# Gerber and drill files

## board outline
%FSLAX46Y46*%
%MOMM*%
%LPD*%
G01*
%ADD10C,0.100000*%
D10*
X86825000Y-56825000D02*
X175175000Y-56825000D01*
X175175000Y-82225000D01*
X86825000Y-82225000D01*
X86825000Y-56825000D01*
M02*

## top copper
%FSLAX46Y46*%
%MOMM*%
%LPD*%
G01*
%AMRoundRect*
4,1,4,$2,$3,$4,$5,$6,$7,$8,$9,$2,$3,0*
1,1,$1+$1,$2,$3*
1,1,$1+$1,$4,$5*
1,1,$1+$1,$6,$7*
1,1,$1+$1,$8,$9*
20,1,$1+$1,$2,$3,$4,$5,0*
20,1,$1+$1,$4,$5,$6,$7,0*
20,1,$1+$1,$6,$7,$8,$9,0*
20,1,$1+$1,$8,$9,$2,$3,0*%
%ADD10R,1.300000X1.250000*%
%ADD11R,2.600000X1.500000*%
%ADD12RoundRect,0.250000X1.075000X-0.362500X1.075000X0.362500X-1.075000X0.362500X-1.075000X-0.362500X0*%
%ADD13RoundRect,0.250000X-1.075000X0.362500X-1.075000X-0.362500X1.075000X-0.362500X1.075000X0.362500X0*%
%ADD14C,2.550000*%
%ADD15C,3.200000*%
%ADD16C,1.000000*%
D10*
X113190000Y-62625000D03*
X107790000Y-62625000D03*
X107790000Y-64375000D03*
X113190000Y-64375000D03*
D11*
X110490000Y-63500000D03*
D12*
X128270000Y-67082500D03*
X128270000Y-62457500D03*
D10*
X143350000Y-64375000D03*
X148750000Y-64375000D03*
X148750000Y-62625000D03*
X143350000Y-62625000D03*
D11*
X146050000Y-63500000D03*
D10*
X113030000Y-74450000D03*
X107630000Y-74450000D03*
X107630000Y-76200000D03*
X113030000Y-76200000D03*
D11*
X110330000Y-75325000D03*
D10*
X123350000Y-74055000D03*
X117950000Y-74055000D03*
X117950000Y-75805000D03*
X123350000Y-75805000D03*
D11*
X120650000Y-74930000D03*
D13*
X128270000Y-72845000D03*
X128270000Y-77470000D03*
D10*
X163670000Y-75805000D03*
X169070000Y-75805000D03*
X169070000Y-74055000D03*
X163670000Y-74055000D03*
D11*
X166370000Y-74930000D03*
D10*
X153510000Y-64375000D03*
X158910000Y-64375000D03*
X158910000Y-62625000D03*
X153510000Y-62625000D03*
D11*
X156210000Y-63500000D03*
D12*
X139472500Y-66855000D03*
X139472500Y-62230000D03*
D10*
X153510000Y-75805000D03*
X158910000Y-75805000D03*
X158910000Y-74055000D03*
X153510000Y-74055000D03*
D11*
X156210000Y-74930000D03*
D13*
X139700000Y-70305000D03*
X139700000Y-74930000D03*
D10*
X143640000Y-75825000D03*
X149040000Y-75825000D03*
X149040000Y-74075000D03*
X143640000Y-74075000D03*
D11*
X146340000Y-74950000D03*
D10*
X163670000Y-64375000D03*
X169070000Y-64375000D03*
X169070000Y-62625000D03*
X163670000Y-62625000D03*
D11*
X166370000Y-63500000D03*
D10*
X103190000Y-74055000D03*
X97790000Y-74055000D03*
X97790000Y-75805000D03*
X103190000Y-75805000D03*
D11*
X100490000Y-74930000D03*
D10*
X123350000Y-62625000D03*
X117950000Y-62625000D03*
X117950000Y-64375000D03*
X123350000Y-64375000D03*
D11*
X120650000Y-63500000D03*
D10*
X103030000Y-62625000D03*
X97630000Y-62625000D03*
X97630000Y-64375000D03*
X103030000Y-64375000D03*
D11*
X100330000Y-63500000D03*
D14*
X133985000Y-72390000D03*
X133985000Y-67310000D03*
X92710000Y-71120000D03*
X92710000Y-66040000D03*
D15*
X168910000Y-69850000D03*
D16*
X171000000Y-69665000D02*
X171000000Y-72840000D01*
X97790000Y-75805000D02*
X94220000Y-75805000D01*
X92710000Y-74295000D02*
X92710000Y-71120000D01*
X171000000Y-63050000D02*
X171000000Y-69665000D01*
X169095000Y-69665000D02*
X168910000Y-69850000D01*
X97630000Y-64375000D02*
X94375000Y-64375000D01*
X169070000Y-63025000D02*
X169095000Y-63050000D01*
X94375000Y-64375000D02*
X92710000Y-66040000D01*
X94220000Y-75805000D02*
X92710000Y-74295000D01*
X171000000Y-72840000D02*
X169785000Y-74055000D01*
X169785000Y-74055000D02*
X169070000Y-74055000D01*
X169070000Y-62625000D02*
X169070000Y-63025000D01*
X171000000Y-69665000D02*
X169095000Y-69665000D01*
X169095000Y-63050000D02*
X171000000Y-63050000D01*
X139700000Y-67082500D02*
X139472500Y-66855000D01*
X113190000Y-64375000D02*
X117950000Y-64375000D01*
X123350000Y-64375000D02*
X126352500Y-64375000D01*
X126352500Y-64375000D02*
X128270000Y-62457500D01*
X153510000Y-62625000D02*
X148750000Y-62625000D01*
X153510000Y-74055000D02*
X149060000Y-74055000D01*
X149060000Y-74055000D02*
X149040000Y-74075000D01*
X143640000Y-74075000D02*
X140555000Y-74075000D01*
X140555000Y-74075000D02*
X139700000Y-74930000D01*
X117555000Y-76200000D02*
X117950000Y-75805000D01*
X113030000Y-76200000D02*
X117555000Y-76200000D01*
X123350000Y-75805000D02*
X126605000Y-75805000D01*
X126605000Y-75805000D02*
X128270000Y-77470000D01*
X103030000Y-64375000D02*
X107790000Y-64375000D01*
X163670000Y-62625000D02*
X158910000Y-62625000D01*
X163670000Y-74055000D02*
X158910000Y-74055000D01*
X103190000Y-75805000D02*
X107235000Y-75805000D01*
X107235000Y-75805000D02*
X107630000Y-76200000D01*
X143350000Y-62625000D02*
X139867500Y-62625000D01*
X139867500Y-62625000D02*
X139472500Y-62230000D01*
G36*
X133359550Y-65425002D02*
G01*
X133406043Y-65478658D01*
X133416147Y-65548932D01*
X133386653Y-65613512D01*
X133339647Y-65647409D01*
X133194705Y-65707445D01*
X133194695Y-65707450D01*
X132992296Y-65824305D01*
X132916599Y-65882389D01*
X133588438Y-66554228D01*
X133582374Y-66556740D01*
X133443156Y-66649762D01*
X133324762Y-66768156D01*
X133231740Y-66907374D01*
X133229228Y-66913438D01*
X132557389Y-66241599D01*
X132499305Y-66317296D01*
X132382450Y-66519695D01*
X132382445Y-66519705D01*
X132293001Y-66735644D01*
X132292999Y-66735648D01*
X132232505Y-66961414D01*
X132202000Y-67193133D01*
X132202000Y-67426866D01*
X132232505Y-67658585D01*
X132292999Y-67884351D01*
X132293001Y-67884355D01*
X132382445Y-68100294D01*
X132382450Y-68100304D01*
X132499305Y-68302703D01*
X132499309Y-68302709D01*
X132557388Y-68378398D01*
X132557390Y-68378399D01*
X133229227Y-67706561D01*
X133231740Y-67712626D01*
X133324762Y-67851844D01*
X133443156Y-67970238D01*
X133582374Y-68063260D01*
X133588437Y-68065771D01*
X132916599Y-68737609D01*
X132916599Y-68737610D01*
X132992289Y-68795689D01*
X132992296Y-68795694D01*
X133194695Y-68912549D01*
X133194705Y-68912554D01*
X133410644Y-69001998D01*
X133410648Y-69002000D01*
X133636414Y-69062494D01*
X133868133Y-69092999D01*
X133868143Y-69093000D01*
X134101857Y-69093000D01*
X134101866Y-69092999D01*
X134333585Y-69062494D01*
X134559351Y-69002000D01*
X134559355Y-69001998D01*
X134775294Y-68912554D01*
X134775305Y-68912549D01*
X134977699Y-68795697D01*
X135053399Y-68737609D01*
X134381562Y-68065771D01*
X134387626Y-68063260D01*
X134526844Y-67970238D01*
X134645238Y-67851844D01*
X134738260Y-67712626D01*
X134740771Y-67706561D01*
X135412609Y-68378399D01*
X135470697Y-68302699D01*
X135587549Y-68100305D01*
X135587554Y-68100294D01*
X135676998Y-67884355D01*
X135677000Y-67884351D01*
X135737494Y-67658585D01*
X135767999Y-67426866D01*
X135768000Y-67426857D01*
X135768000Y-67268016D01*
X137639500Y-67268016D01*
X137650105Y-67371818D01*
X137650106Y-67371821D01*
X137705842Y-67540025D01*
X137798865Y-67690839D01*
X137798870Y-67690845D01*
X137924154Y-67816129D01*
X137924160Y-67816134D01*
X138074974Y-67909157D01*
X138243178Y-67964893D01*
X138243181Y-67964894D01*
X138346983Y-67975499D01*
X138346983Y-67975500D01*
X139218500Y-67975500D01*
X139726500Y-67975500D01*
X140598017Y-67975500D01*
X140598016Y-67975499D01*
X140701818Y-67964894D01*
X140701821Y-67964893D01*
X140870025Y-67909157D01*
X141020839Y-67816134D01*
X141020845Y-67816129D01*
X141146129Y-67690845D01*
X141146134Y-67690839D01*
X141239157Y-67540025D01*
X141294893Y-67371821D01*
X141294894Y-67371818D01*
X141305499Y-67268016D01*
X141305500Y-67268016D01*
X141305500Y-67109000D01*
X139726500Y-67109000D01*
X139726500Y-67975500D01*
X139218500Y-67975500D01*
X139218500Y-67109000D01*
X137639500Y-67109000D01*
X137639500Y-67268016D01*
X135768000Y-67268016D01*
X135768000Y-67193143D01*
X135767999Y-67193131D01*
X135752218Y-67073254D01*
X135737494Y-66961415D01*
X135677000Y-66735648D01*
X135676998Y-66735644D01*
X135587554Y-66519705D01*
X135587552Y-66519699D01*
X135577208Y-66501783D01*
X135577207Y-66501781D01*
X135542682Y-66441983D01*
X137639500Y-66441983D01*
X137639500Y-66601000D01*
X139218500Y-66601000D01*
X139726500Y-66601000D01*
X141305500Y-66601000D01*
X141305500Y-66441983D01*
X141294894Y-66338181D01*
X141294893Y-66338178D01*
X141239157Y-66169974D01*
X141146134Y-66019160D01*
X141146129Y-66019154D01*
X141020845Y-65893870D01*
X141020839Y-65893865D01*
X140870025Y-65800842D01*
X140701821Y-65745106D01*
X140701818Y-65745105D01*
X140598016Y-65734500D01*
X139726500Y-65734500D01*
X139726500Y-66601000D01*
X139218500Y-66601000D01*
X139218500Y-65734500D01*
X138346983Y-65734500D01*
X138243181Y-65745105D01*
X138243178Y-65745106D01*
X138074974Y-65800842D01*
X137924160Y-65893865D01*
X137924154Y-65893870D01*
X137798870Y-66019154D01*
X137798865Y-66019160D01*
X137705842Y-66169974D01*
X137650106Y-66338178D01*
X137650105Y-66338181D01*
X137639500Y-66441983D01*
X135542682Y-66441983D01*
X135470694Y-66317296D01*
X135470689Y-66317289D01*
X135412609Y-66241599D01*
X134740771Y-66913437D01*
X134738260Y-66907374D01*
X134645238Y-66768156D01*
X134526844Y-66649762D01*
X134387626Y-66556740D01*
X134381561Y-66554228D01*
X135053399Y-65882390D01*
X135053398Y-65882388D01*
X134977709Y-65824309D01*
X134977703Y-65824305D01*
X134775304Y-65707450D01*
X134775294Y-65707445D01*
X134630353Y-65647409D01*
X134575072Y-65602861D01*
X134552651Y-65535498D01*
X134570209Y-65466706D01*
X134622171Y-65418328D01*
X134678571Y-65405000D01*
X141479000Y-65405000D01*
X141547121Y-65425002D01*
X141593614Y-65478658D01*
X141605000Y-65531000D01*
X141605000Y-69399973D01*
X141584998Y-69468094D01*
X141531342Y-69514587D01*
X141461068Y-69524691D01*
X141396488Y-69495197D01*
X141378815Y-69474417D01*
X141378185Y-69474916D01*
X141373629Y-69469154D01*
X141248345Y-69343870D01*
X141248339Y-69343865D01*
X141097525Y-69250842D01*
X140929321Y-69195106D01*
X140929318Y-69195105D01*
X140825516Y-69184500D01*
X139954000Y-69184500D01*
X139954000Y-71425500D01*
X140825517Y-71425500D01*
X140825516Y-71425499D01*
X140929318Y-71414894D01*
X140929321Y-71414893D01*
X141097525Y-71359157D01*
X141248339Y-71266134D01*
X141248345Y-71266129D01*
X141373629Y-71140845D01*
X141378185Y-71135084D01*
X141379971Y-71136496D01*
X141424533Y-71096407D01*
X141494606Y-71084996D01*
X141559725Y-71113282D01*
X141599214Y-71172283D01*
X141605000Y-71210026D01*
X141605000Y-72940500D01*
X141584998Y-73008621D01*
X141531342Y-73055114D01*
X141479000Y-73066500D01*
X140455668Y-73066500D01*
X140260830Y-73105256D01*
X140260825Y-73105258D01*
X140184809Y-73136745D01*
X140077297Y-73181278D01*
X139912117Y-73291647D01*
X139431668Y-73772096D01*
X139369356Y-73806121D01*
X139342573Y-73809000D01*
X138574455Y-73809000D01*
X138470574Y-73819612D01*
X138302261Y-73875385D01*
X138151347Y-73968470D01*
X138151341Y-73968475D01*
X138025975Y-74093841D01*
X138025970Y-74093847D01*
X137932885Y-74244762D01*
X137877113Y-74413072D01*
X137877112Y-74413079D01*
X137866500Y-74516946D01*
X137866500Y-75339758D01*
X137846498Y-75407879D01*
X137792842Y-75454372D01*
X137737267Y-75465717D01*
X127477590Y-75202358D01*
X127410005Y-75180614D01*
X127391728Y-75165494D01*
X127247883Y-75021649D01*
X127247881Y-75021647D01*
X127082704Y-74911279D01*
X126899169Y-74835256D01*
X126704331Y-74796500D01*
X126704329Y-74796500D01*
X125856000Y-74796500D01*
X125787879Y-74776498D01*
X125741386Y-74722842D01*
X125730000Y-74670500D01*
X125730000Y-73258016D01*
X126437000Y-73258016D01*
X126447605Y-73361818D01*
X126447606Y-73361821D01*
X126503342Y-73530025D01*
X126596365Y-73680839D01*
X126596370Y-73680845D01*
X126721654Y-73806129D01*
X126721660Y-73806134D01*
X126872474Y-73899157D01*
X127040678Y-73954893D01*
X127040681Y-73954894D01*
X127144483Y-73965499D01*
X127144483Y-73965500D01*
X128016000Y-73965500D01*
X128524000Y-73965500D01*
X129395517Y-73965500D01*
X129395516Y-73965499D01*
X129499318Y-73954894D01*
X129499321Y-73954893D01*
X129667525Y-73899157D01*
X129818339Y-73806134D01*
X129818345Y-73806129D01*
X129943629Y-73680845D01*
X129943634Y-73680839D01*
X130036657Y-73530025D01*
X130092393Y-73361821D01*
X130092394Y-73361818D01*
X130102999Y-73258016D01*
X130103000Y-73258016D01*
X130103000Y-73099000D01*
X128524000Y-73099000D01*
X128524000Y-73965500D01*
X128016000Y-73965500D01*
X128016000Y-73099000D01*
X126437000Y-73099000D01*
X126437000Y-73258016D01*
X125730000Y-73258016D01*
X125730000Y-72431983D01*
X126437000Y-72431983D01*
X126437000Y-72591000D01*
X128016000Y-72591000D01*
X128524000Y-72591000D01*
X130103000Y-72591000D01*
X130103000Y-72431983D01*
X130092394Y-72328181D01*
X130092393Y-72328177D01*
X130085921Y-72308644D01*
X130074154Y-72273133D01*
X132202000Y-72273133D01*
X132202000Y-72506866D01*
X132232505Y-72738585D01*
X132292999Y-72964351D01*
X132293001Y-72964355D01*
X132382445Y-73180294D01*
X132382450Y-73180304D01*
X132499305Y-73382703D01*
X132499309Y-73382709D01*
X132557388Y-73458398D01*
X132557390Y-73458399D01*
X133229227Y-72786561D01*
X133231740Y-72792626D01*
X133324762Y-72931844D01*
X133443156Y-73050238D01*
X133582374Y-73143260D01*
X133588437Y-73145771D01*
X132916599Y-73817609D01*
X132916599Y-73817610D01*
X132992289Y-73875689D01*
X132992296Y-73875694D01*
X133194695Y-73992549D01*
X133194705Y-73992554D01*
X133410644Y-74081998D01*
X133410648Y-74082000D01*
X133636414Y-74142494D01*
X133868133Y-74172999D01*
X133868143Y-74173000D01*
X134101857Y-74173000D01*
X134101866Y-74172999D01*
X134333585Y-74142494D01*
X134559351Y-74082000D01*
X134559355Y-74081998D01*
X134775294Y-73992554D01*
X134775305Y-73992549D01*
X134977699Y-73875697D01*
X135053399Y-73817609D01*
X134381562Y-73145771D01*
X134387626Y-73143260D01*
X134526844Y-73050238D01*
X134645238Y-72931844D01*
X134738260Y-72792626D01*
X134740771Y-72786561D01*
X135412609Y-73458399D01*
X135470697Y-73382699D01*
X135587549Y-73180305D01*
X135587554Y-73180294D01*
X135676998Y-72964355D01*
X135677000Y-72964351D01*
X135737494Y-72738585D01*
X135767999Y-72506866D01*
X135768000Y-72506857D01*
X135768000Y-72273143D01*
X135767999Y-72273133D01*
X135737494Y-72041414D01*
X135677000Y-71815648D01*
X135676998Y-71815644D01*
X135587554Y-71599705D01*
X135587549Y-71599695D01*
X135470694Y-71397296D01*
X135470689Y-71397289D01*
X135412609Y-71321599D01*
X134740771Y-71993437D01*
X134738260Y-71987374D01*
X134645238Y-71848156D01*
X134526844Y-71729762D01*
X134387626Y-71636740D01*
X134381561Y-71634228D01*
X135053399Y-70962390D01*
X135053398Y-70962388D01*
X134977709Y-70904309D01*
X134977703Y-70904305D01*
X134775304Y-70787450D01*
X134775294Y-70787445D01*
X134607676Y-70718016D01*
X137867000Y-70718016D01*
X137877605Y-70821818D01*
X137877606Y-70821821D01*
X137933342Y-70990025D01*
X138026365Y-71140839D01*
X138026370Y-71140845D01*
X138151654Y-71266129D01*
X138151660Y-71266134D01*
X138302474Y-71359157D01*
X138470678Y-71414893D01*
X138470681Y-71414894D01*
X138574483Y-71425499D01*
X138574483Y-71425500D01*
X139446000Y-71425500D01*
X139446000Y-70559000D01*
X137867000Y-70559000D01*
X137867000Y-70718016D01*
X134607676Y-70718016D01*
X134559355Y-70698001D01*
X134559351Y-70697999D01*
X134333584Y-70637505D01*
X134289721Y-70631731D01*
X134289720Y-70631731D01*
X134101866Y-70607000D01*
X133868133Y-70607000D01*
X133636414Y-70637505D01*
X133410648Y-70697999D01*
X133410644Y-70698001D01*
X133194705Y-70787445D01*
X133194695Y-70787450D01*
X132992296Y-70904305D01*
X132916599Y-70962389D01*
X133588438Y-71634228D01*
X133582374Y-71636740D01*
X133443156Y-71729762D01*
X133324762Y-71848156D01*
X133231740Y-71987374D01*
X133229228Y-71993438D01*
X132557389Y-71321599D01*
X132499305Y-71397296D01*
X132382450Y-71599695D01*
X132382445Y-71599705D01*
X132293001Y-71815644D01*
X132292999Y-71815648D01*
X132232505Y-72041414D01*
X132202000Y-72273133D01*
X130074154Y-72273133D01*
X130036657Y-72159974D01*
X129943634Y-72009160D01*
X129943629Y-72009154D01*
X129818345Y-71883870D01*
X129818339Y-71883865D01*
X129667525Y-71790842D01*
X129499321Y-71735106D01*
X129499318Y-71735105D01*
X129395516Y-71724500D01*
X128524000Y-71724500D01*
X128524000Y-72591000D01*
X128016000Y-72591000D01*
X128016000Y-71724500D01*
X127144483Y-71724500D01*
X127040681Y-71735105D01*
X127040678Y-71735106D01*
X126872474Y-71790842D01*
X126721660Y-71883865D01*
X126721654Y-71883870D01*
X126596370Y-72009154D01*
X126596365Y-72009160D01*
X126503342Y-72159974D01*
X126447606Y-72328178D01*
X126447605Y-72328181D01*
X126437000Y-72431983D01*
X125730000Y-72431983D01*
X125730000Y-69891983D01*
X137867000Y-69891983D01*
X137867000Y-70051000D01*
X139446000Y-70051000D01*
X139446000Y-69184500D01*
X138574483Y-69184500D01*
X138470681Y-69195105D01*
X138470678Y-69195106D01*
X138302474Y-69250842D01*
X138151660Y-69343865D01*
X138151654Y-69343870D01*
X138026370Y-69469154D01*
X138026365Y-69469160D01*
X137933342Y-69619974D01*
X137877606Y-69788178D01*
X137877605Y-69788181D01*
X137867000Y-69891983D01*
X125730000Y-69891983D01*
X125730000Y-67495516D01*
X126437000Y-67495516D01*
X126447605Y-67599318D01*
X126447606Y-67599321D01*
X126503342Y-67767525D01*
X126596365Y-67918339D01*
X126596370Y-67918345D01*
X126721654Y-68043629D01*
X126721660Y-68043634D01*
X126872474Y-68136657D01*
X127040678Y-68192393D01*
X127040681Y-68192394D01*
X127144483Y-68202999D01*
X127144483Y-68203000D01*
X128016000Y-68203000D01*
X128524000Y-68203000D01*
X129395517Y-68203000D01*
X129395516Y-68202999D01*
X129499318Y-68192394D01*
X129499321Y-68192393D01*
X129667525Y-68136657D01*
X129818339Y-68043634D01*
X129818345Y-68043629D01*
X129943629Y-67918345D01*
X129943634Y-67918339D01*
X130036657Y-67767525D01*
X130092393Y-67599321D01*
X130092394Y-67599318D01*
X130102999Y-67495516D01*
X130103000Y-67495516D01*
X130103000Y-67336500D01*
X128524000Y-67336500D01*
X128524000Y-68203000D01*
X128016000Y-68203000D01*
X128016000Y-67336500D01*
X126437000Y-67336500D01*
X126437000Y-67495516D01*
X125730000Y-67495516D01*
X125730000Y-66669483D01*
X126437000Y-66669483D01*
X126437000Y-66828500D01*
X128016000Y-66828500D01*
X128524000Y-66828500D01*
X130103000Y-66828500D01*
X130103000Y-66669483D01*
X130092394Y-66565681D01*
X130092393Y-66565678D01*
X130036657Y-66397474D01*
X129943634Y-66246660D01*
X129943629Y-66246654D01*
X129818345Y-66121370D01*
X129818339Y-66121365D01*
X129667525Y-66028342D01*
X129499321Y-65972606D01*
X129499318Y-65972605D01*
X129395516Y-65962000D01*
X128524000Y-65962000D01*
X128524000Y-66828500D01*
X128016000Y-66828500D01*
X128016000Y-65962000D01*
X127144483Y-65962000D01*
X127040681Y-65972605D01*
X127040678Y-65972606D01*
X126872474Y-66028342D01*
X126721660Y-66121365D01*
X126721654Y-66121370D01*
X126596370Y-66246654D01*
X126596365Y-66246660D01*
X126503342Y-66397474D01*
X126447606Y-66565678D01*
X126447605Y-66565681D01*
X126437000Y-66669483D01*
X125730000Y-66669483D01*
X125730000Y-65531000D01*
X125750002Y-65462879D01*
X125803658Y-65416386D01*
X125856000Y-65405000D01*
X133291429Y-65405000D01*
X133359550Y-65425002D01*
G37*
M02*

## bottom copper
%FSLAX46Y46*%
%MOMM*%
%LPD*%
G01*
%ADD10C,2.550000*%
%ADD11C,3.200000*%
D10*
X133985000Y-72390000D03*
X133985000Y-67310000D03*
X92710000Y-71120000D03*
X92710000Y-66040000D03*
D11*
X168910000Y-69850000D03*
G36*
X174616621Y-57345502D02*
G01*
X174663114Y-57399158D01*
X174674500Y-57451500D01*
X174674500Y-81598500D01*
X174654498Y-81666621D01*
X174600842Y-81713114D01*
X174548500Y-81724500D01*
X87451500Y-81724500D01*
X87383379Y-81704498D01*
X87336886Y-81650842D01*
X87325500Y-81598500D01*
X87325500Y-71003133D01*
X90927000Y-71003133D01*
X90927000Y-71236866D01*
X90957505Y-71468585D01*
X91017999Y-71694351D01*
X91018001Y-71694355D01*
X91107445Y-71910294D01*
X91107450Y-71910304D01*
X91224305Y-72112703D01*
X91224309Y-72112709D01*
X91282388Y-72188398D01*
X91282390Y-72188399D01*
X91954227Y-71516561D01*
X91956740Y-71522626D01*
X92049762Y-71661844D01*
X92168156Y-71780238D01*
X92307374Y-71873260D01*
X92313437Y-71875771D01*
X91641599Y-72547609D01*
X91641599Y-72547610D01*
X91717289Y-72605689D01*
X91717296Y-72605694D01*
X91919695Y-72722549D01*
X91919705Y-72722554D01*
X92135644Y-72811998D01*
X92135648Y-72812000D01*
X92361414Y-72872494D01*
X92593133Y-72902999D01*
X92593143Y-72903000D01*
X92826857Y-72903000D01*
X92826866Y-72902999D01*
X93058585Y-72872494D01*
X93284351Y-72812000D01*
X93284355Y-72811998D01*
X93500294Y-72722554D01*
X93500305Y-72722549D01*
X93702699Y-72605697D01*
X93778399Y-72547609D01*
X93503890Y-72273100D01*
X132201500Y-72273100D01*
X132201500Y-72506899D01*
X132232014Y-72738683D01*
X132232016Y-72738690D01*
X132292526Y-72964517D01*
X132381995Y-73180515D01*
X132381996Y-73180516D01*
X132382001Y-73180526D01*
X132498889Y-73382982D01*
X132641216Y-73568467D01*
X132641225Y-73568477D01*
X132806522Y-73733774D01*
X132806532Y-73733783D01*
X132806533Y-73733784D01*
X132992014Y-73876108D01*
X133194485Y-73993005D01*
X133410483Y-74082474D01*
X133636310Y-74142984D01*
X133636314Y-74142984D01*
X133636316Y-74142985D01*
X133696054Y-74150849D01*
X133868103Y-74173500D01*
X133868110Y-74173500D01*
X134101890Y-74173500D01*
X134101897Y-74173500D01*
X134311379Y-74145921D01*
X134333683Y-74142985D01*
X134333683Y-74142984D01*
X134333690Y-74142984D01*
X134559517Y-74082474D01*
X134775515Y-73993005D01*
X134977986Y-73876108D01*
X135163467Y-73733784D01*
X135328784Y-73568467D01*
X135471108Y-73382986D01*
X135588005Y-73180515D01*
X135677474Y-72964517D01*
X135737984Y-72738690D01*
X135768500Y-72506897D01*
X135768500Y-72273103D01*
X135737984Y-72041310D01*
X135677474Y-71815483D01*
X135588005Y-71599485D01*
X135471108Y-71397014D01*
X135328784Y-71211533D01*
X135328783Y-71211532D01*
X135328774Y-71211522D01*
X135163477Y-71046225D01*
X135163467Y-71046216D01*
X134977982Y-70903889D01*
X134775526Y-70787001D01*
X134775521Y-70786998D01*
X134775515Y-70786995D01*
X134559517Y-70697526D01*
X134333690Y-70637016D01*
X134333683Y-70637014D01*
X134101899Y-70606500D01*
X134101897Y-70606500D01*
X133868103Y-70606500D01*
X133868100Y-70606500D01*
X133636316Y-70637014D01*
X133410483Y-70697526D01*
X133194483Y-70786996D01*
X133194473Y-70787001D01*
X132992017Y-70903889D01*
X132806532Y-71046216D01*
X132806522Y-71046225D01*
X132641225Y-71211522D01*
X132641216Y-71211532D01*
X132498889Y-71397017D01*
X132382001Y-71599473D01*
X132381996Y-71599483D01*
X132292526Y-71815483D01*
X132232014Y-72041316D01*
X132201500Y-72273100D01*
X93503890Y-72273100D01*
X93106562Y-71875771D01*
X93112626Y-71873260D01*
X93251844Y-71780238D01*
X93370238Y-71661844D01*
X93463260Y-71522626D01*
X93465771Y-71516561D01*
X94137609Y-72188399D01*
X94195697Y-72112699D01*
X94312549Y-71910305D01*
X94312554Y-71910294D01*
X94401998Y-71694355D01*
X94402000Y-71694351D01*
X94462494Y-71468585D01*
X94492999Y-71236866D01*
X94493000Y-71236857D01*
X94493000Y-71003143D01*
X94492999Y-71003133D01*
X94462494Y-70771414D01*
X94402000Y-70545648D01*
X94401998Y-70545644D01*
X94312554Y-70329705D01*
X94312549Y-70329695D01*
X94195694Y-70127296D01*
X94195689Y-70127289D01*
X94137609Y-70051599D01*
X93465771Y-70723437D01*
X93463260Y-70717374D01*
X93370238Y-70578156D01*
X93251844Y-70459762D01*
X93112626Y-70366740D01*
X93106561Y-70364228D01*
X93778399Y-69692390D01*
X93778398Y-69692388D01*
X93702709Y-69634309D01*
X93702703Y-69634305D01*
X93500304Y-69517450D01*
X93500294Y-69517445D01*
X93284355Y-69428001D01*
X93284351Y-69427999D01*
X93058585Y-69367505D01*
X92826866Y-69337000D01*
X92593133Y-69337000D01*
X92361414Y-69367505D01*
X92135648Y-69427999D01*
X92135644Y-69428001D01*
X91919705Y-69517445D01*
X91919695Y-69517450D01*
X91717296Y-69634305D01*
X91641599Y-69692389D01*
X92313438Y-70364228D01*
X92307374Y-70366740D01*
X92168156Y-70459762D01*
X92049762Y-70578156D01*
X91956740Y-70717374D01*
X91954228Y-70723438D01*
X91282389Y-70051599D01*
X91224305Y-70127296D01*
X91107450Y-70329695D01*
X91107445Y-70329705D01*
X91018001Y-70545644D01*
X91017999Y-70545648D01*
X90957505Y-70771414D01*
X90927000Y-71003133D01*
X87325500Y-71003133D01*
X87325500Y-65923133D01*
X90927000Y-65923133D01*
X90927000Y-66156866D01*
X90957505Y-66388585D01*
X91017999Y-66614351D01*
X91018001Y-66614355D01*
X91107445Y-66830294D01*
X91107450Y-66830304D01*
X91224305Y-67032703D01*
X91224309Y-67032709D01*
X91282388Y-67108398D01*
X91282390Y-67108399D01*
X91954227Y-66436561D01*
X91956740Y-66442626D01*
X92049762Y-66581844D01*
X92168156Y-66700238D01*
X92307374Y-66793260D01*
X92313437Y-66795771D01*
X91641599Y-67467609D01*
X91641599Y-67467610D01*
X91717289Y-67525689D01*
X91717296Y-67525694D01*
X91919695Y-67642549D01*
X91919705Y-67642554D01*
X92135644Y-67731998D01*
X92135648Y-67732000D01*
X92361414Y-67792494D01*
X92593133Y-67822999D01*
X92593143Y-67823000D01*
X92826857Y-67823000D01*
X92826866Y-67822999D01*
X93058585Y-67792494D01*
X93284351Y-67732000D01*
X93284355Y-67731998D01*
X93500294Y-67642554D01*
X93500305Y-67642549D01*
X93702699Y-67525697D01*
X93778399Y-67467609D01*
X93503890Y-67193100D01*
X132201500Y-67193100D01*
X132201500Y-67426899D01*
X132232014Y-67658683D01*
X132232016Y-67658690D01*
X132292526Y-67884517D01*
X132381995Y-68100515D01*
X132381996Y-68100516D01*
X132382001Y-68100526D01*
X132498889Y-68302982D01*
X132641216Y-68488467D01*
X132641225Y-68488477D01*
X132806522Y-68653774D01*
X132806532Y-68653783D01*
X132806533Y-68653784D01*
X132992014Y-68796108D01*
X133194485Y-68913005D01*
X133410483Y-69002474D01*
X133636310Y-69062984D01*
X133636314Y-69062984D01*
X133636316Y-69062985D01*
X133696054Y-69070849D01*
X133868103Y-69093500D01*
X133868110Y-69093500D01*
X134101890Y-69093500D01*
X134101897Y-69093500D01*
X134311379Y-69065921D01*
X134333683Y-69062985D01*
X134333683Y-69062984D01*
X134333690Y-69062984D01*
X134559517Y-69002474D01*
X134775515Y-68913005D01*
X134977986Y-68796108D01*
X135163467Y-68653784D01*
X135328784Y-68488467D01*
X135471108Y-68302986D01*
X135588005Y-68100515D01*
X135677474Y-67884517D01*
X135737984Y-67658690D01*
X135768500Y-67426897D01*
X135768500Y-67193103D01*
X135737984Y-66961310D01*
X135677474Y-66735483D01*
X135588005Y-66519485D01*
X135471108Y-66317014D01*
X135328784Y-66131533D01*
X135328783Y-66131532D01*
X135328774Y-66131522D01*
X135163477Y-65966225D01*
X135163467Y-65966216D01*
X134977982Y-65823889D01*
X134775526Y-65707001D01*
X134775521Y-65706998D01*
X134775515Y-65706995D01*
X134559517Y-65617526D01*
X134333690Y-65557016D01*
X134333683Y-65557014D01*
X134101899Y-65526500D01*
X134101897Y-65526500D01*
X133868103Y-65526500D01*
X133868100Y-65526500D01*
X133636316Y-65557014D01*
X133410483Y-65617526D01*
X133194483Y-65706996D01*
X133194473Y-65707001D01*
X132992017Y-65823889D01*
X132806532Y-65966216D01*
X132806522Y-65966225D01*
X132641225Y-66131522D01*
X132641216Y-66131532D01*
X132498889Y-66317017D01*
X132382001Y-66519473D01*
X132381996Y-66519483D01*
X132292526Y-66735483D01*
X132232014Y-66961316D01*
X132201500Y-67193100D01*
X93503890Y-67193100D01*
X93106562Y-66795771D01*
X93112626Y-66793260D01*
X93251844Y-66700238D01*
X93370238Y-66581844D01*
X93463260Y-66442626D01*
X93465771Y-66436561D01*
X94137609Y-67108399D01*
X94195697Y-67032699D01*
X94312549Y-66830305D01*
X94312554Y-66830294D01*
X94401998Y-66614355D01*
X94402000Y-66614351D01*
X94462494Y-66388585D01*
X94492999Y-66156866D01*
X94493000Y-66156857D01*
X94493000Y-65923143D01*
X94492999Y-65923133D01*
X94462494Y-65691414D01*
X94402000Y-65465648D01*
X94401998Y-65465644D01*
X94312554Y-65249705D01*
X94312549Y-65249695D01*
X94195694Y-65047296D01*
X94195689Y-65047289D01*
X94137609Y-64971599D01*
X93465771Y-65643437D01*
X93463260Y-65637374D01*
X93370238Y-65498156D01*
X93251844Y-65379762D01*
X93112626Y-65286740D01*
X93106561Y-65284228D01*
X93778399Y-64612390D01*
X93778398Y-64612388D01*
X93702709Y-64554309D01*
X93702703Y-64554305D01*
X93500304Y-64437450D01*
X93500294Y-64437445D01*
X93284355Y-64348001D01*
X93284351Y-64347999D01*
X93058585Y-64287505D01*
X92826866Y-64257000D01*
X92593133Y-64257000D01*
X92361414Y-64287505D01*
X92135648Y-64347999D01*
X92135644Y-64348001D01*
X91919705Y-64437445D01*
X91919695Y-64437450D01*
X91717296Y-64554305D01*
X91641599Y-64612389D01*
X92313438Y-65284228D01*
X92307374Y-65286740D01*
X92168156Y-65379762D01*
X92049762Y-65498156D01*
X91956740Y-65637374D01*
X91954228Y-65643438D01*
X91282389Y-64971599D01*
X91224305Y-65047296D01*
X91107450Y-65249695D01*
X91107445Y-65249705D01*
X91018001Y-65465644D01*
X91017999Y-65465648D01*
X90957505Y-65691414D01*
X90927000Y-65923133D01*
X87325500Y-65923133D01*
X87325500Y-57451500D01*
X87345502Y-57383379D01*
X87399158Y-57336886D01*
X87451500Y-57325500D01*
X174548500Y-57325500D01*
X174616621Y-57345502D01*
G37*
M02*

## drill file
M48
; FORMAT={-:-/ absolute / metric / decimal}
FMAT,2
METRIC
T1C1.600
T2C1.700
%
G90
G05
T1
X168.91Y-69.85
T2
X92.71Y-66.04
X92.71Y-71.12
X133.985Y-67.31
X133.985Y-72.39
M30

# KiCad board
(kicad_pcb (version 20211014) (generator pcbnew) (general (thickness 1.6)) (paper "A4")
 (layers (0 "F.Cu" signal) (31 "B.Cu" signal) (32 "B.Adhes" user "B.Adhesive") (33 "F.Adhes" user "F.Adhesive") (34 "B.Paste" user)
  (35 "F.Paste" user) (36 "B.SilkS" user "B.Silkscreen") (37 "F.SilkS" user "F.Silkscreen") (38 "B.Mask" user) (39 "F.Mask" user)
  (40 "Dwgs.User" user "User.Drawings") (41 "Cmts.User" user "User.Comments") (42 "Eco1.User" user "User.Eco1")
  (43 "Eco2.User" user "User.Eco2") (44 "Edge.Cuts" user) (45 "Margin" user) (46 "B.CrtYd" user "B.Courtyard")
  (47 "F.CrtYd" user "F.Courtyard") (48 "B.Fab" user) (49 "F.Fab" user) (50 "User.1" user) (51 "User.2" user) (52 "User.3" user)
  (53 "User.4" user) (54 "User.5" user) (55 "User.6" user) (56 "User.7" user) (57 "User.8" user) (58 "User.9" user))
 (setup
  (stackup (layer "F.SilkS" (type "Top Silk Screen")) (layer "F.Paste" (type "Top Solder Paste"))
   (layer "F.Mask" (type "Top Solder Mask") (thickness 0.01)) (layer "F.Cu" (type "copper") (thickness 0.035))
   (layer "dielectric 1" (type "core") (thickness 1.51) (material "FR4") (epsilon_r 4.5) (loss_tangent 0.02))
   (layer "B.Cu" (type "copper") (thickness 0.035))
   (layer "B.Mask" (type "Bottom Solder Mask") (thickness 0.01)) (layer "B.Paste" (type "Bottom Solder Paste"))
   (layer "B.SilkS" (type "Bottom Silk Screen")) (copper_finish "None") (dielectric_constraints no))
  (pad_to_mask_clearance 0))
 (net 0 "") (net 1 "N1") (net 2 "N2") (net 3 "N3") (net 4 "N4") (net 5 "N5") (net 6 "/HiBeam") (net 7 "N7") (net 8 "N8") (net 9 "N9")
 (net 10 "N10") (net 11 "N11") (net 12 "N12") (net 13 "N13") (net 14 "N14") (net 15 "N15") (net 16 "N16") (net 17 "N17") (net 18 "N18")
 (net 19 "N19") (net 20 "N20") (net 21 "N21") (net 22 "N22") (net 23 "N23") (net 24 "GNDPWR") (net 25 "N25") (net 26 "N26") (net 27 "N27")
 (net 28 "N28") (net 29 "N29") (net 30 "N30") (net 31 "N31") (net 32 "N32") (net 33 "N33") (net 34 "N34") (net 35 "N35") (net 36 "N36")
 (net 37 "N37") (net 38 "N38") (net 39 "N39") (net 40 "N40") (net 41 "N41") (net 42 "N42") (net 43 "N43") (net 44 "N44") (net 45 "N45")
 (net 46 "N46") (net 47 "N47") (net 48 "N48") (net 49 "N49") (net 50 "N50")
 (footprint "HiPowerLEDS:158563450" (layer "F.Cu") (at 110.49 63.5 180)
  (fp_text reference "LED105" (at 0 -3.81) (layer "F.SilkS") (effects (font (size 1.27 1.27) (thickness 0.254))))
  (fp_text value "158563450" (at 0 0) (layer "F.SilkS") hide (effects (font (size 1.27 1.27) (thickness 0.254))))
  (pad "1" smd rect locked (at -2.7 0.875 270) (size 1.25 1.3) (layers "F.Cu" "F.Paste" "F.Mask") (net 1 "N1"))
  (pad "2" smd rect locked (at 2.7 0.875 270) (size 1.25 1.3) (layers "F.Cu" "F.Paste" "F.Mask") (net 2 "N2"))
  (pad "3" smd rect locked (at 2.7 -0.875 270) (size 1.25 1.3) (layers "F.Cu" "F.Paste" "F.Mask") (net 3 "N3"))
  (pad "4" smd rect locked (at -2.7 -0.875 270) (size 1.25 1.3) (layers "F.Cu" "F.Paste" "F.Mask") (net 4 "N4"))
  (pad "5" smd rect locked (at 0 0 270) (size 1.5 2.6) (layers "F.Cu" "F.Paste" "F.Mask") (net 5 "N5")))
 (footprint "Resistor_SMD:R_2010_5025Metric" (layer "F.Cu") (at 128.27 64.77 90)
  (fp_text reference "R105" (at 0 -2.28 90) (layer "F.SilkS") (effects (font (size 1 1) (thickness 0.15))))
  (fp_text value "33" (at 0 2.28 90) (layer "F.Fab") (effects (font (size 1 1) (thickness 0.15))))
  (pad "1" smd roundrect (at -2.3125 0 90) (size 1.225 2.65) (layers "F.Cu" "F.Paste" "F.Mask") (roundrect_rratio 0.204082)
   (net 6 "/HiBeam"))
  (pad "2" smd roundrect (at 2.3125 0 90) (size 1.225 2.65) (layers "F.Cu" "F.Paste" "F.Mask") (roundrect_rratio 0.204082) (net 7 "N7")))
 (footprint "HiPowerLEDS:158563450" (layer "F.Cu") (at 146.05 63.5)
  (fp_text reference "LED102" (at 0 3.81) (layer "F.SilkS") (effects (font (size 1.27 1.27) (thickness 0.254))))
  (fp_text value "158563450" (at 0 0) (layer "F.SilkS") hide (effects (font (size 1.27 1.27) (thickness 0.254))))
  (pad "1" smd rect locked (at -2.7 0.875 90) (size 1.25 1.3) (layers "F.Cu" "F.Paste" "F.Mask") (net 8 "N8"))
  (pad "2" smd rect locked (at 2.7 0.875 90) (size 1.25 1.3) (layers "F.Cu" "F.Paste" "F.Mask") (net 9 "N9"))
  (pad "3" smd rect locked (at 2.7 -0.875 90) (size 1.25 1.3) (layers "F.Cu" "F.Paste" "F.Mask") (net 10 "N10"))
  (pad "4" smd rect locked (at -2.7 -0.875 90) (size 1.25 1.3) (layers "F.Cu" "F.Paste" "F.Mask") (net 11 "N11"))
  (pad "5" smd rect locked (at 0 0 90) (size 1.5 2.6) (layers "F.Cu" "F.Paste" "F.Mask") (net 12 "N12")))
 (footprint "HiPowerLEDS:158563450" (layer "F.Cu") (at 110.33 75.325 180)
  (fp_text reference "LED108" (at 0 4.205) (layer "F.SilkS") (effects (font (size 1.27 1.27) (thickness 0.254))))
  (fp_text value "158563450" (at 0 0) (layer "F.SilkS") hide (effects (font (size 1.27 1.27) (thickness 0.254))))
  (pad "1" smd rect locked (at -2.7 0.875 270) (size 1.25 1.3) (layers "F.Cu" "F.Paste" "F.Mask") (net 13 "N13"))
  (pad "2" smd rect locked (at 2.7 0.875 270) (size 1.25 1.3) (layers "F.Cu" "F.Paste" "F.Mask") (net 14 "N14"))
  (pad "3" smd rect locked (at 2.7 -0.875 270) (size 1.25 1.3) (layers "F.Cu" "F.Paste" "F.Mask") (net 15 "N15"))
  (pad "4" smd rect locked (at -2.7 -0.875 270) (size 1.25 1.3) (layers "F.Cu" "F.Paste" "F.Mask") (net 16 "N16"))
  (pad "5" smd rect locked (at 0 0 270) (size 1.5 2.6) (layers "F.Cu" "F.Paste" "F.Mask") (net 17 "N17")))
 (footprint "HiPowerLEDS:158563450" (layer "F.Cu") (at 120.65 74.93 180)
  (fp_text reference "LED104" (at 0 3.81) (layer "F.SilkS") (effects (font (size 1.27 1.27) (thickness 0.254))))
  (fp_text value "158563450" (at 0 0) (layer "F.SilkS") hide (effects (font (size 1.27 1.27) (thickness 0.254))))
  (pad "1" smd rect locked (at -2.7 0.875 270) (size 1.25 1.3) (layers "F.Cu" "F.Paste" "F.Mask") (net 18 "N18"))
  (pad "2" smd rect locked (at 2.7 0.875 270) (size 1.25 1.3) (layers "F.Cu" "F.Paste" "F.Mask") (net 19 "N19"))
  (pad "3" smd rect locked (at 2.7 -0.875 270) (size 1.25 1.3) (layers "F.Cu" "F.Paste" "F.Mask") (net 16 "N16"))
  (pad "4" smd rect locked (at -2.7 -0.875 270) (size 1.25 1.3) (layers "F.Cu" "F.Paste" "F.Mask") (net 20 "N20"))
  (pad "5" smd rect locked (at 0 0 270) (size 1.5 2.6) (layers "F.Cu" "F.Paste" "F.Mask") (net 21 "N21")))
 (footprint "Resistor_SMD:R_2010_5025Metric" (layer "F.Cu") (at 128.27 75.1575 -90)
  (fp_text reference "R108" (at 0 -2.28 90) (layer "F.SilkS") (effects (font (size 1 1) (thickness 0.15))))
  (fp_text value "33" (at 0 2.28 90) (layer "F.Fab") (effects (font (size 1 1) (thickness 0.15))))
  (pad "1" smd roundrect (at -2.3125 0 270) (size 1.225 2.65) (layers "F.Cu" "F.Paste" "F.Mask") (roundrect_rratio 0.204082)
   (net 6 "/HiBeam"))
  (pad "2" smd roundrect (at 2.3125 0 270) (size 1.225 2.65) (layers "F.Cu" "F.Paste" "F.Mask") (roundrect_rratio 0.204082) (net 20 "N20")))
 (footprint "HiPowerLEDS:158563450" (layer "F.Cu") (at 166.37 74.93)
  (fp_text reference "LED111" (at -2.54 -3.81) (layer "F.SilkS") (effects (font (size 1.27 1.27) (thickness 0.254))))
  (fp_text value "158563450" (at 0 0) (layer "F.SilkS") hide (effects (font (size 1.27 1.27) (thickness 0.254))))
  (pad "1" smd rect locked (at -2.7 0.875 90) (size 1.25 1.3) (layers "F.Cu" "F.Paste" "F.Mask") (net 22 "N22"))
  (pad "2" smd rect locked (at 2.7 0.875 90) (size 1.25 1.3) (layers "F.Cu" "F.Paste" "F.Mask") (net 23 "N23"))
  (pad "3" smd rect locked (at 2.7 -0.875 90) (size 1.25 1.3) (layers "F.Cu" "F.Paste" "F.Mask") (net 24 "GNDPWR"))
  (pad "4" smd rect locked (at -2.7 -0.875 90) (size 1.25 1.3) (layers "F.Cu" "F.Paste" "F.Mask") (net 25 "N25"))
  (pad "5" smd rect locked (at 0 0 90) (size 1.5 2.6) (layers "F.Cu" "F.Paste" "F.Mask") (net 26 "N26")))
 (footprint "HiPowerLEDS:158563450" (layer "F.Cu") (at 156.21 63.5)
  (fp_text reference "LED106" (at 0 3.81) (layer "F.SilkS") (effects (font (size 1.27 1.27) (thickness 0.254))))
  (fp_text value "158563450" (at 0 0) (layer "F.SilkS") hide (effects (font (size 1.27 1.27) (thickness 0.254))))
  (pad "1" smd rect locked (at -2.7 0.875 90) (size 1.25 1.3) (layers "F.Cu" "F.Paste" "F.Mask") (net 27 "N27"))
  (pad "2" smd rect locked (at 2.7 0.875 90) (size 1.25 1.3) (layers "F.Cu" "F.Paste" "F.Mask") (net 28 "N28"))
  (pad "3" smd rect locked (at 2.7 -0.875 90) (size 1.25 1.3) (layers "F.Cu" "F.Paste" "F.Mask") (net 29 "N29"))
  (pad "4" smd rect locked (at -2.7 -0.875 90) (size 1.25 1.3) (layers "F.Cu" "F.Paste" "F.Mask") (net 10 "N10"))
  (pad "5" smd rect locked (at 0 0 90) (size 1.5 2.6) (layers "F.Cu" "F.Paste" "F.Mask") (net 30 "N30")))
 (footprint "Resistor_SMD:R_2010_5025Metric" (layer "F.Cu") (at 139.4725 64.5425 90)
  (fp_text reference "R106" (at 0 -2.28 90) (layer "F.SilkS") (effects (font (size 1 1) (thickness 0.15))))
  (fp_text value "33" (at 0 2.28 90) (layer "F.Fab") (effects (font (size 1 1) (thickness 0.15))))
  (pad "1" smd roundrect (at -2.3125 0 90) (size 1.225 2.65) (layers "F.Cu" "F.Paste" "F.Mask") (roundrect_rratio 0.204082)
   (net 6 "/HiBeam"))
  (pad "2" smd roundrect (at 2.3125 0 90) (size 1.225 2.65) (layers "F.Cu" "F.Paste" "F.Mask") (roundrect_rratio 0.204082) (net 11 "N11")))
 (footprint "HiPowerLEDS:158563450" (layer "F.Cu") (at 156.21 74.93)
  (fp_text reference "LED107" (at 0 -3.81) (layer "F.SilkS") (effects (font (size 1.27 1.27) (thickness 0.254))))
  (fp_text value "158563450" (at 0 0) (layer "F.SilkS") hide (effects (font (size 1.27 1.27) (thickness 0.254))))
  (pad "1" smd rect locked (at -2.7 0.875 90) (size 1.25 1.3) (layers "F.Cu" "F.Paste" "F.Mask") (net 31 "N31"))
  (pad "2" smd rect locked (at 2.7 0.875 90) (size 1.25 1.3) (layers "F.Cu" "F.Paste" "F.Mask") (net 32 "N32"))
  (pad "3" smd rect locked (at 2.7 -0.875 90) (size 1.25 1.3) (layers "F.Cu" "F.Paste" "F.Mask") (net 25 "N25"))
  (pad "4" smd rect locked (at -2.7 -0.875 90) (size 1.25 1.3) (layers "F.Cu" "F.Paste" "F.Mask") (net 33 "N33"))
  (pad "5" smd rect locked (at 0 0 90) (size 1.5 2.6) (layers "F.Cu" "F.Paste" "F.Mask") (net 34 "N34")))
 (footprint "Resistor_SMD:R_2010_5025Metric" (layer "F.Cu") (at 139.7 72.6175 -90)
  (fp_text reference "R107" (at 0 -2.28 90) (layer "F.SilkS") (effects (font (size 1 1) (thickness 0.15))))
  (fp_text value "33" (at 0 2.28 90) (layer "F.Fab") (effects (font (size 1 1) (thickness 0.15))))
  (pad "1" smd roundrect (at -2.3125 0 270) (size 1.225 2.65) (layers "F.Cu" "F.Paste" "F.Mask") (roundrect_rratio 0.204082)
   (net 6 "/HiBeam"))
  (pad "2" smd roundrect (at 2.3125 0 270) (size 1.225 2.65) (layers "F.Cu" "F.Paste" "F.Mask") (roundrect_rratio 0.204082) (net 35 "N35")))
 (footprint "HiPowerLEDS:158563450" (layer "F.Cu") (at 146.34 74.95)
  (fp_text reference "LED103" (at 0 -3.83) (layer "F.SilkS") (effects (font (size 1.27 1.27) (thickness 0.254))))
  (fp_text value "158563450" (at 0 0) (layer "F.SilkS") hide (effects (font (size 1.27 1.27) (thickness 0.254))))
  (pad "1" smd rect locked (at -2.7 0.875 90) (size 1.25 1.3) (layers "F.Cu" "F.Paste" "F.Mask") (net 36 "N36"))
  (pad "2" smd rect locked (at 2.7 0.875 90) (size 1.25 1.3) (layers "F.Cu" "F.Paste" "F.Mask") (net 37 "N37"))
  (pad "3" smd rect locked (at 2.7 -0.875 90) (size 1.25 1.3) (layers "F.Cu" "F.Paste" "F.Mask") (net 33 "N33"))
  (pad "4" smd rect locked (at -2.7 -0.875 90) (size 1.25 1.3) (layers "F.Cu" "F.Paste" "F.Mask") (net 35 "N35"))
  (pad "5" smd rect locked (at 0 0 90) (size 1.5 2.6) (layers "F.Cu" "F.Paste" "F.Mask") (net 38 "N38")))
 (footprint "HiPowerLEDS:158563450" (layer "F.Cu") (at 166.37 63.5)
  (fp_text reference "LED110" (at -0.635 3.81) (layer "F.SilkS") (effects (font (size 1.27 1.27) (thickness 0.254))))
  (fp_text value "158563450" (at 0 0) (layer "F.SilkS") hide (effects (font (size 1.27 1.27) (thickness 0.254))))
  (pad "1" smd rect locked (at -2.7 0.875 90) (size 1.25 1.3) (layers "F.Cu" "F.Paste" "F.Mask") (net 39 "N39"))
  (pad "2" smd rect locked (at 2.7 0.875 90) (size 1.25 1.3) (layers "F.Cu" "F.Paste" "F.Mask") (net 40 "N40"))
  (pad "3" smd rect locked (at 2.7 -0.875 90) (size 1.25 1.3) (layers "F.Cu" "F.Paste" "F.Mask") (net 24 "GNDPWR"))
  (pad "4" smd rect locked (at -2.7 -0.875 90) (size 1.25 1.3) (layers "F.Cu" "F.Paste" "F.Mask") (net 29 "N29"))
  (pad "5" smd rect locked (at 0 0 90) (size 1.5 2.6) (layers "F.Cu" "F.Paste" "F.Mask") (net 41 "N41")))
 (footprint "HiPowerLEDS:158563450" (layer "F.Cu") (at 100.49 74.93 180)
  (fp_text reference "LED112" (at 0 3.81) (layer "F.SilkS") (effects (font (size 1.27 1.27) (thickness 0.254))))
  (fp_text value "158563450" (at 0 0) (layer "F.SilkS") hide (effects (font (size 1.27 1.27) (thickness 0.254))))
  (pad "1" smd rect locked (at -2.7 0.875 270) (size 1.25 1.3) (layers "F.Cu" "F.Paste" "F.Mask") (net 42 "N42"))
  (pad "2" smd rect locked (at 2.7 0.875 270) (size 1.25 1.3) (layers "F.Cu" "F.Paste" "F.Mask") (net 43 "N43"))
  (pad "3" smd rect locked (at 2.7 -0.875 270) (size 1.25 1.3) (layers "F.Cu" "F.Paste" "F.Mask") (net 24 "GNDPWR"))
  (pad "4" smd rect locked (at -2.7 -0.875 270) (size 1.25 1.3) (layers "F.Cu" "F.Paste" "F.Mask") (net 15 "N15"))
  (pad "5" smd rect locked (at 0 0 270) (size 1.5 2.6) (layers "F.Cu" "F.Paste" "F.Mask") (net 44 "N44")))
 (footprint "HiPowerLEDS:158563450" (layer "F.Cu") (at 120.65 63.5 180)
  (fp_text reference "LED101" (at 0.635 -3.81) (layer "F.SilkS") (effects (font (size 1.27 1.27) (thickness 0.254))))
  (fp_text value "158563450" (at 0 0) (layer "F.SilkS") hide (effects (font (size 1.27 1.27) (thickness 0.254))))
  (pad "1" smd rect locked (at -2.7 0.875 270) (size 1.25 1.3) (layers "F.Cu" "F.Paste" "F.Mask") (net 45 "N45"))
  (pad "2" smd rect locked (at 2.7 0.875 270) (size 1.25 1.3) (layers "F.Cu" "F.Paste" "F.Mask") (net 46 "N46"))
  (pad "3" smd rect locked (at 2.7 -0.875 270) (size 1.25 1.3) (layers "F.Cu" "F.Paste" "F.Mask") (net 4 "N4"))
  (pad "4" smd rect locked (at -2.7 -0.875 270) (size 1.25 1.3) (layers "F.Cu" "F.Paste" "F.Mask") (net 7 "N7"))
  (pad "5" smd rect locked (at 0 0 270) (size 1.5 2.6) (layers "F.Cu" "F.Paste" "F.Mask") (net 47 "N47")))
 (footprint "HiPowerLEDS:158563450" (layer "F.Cu") (at 100.33 63.5 180)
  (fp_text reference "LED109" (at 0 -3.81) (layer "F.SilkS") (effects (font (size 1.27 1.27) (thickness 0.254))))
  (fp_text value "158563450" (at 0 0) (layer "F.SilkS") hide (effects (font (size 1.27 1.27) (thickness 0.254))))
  (pad "1" smd rect locked (at -2.7 0.875 270) (size 1.25 1.3) (layers "F.Cu" "F.Paste" "F.Mask") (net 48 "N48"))
  (pad "2" smd rect locked (at 2.7 0.875 270) (size 1.25 1.3) (layers "F.Cu" "F.Paste" "F.Mask") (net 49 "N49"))
  (pad "3" smd rect locked (at 2.7 -0.875 270) (size 1.25 1.3) (layers "F.Cu" "F.Paste" "F.Mask") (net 24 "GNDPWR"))
  (pad "4" smd rect locked (at -2.7 -0.875 270) (size 1.25 1.3) (layers "F.Cu" "F.Paste" "F.Mask") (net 3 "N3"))
  (pad "5" smd rect locked (at 0 0 270) (size 1.5 2.6) (layers "F.Cu" "F.Paste" "F.Mask") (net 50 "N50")))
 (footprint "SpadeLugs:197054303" (layer "B.Cu") (at 133.985 72.39 90)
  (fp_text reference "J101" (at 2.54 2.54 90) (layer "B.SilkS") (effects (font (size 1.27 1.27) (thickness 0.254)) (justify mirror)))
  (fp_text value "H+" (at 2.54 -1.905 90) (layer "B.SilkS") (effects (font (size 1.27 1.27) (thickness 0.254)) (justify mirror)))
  (pad "1" thru_hole circle locked (at 0 0 90) (size 2.55 2.55) (drill 1.7) (layers *.Cu *.Mask) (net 6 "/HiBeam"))
  (pad "2" thru_hole circle locked (at 5.08 0 90) (size 2.55 2.55) (drill 1.7) (layers *.Cu *.Mask) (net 6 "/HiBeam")))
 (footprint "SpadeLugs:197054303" (layer "B.Cu") (at 92.71 71.12 90)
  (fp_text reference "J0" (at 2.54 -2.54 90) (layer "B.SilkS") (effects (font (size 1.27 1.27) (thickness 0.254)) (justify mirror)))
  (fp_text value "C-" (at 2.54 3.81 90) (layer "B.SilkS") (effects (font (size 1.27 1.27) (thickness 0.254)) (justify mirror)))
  (pad "1" thru_hole circle locked (at 0 0 90) (size 2.55 2.55) (drill 1.7) (layers *.Cu *.Mask) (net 24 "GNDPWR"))
  (pad "2" thru_hole circle locked (at 5.08 0 90) (size 2.55 2.55) (drill 1.7) (layers *.Cu *.Mask) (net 24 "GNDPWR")))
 (gr_rect (start 86.825 56.825) (end 175.175 82.225) (layer "Edge.Cuts") (width 0.1) (fill none))
 (segment (start 171 69.665) (end 171 72.84) (width 1) (layer "F.Cu") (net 24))
 (segment (start 97.79 75.805) (end 94.22 75.805) (width 1) (layer "F.Cu") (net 24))
 (segment (start 92.71 74.295) (end 92.71 71.12) (width 1) (layer "F.Cu") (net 24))
 (segment (start 171 63.05) (end 171 69.665) (width 1) (layer "F.Cu") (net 24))
 (segment (start 169.095 69.665) (end 168.91 69.85) (width 1) (layer "F.Cu") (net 24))
 (segment (start 97.63 64.375) (end 94.375 64.375) (width 1) (layer "F.Cu") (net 24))
 (segment (start 169.07 63.025) (end 169.095 63.05) (width 1) (layer "F.Cu") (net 24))
 (segment (start 94.375 64.375) (end 92.71 66.04) (width 1) (layer "F.Cu") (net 24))
 (segment (start 94.22 75.805) (end 92.71 74.295) (width 1) (layer "F.Cu") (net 24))
 (segment (start 171 72.84) (end 169.785 74.055) (width 1) (layer "F.Cu") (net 24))
 (segment (start 169.785 74.055) (end 169.07 74.055) (width 1) (layer "F.Cu") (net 24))
 (segment (start 169.07 62.625) (end 169.07 63.025) (width 1) (layer "F.Cu") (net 24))
 (segment (start 171 69.665) (end 169.095 69.665) (width 1) (layer "F.Cu") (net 24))
 (segment (start 169.095 63.05) (end 171 63.05) (width 1) (layer "F.Cu") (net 24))
 (via (at 168.91 69.85) (size 3.2) (drill 1.6) (layers "F.Cu" "B.Cu") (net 24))
 (segment (start 139.7 67.0825) (end 139.4725 66.855) (width 1) (layer "F.Cu") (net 6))
 (segment (start 113.19 64.375) (end 117.95 64.375) (width 1) (layer "F.Cu") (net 4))
 (segment (start 123.35 64.375) (end 126.3525 64.375) (width 1) (layer "F.Cu") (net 7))
 (segment (start 126.3525 64.375) (end 128.27 62.4575) (width 1) (layer "F.Cu") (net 7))
 (segment (start 153.51 62.625) (end 148.75 62.625) (width 1) (layer "F.Cu") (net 10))
 (segment (start 153.51 74.055) (end 149.06 74.055) (width 1) (layer "F.Cu") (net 33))
 (segment (start 149.06 74.055) (end 149.04 74.075) (width 1) (layer "F.Cu") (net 33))
 (segment (start 143.64 74.075) (end 140.555 74.075) (width 1) (layer "F.Cu") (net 35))
 (segment (start 140.555 74.075) (end 139.7 74.93) (width 1) (layer "F.Cu") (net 35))
 (segment (start 117.555 76.2) (end 117.95 75.805) (width 1) (layer "F.Cu") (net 16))
 (segment (start 113.03 76.2) (end 117.555 76.2) (width 1) (layer "F.Cu") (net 16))
 (segment (start 123.35 75.805) (end 126.605 75.805) (width 1) (layer "F.Cu") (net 20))
 (segment (start 126.605 75.805) (end 128.27 77.47) (width 1) (layer "F.Cu") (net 20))
 (segment (start 103.03 64.375) (end 107.79 64.375) (width 1) (layer "F.Cu") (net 3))
 (segment (start 163.67 62.625) (end 158.91 62.625) (width 1) (layer "F.Cu") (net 29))
 (segment (start 163.67 74.055) (end 158.91 74.055) (width 1) (layer "F.Cu") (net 25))
 (segment (start 103.19 75.805) (end 107.235 75.805) (width 1) (layer "F.Cu") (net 15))
 (segment (start 107.235 75.805) (end 107.63 76.2) (width 1) (layer "F.Cu") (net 15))
 (segment (start 143.35 62.625) (end 139.8675 62.625) (width 1) (layer "F.Cu") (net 11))
 (segment (start 139.8675 62.625) (end 139.4725 62.23) (width 1) (layer "F.Cu") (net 11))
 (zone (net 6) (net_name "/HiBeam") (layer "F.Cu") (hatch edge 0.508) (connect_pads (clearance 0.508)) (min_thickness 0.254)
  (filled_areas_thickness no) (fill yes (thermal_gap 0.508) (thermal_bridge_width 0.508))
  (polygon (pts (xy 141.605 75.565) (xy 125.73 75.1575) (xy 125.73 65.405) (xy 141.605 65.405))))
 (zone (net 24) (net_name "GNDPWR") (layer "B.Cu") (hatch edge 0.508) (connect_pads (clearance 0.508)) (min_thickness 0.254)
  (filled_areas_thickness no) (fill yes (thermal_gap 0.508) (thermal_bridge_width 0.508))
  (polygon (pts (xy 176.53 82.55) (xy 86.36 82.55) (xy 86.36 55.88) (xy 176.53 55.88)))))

